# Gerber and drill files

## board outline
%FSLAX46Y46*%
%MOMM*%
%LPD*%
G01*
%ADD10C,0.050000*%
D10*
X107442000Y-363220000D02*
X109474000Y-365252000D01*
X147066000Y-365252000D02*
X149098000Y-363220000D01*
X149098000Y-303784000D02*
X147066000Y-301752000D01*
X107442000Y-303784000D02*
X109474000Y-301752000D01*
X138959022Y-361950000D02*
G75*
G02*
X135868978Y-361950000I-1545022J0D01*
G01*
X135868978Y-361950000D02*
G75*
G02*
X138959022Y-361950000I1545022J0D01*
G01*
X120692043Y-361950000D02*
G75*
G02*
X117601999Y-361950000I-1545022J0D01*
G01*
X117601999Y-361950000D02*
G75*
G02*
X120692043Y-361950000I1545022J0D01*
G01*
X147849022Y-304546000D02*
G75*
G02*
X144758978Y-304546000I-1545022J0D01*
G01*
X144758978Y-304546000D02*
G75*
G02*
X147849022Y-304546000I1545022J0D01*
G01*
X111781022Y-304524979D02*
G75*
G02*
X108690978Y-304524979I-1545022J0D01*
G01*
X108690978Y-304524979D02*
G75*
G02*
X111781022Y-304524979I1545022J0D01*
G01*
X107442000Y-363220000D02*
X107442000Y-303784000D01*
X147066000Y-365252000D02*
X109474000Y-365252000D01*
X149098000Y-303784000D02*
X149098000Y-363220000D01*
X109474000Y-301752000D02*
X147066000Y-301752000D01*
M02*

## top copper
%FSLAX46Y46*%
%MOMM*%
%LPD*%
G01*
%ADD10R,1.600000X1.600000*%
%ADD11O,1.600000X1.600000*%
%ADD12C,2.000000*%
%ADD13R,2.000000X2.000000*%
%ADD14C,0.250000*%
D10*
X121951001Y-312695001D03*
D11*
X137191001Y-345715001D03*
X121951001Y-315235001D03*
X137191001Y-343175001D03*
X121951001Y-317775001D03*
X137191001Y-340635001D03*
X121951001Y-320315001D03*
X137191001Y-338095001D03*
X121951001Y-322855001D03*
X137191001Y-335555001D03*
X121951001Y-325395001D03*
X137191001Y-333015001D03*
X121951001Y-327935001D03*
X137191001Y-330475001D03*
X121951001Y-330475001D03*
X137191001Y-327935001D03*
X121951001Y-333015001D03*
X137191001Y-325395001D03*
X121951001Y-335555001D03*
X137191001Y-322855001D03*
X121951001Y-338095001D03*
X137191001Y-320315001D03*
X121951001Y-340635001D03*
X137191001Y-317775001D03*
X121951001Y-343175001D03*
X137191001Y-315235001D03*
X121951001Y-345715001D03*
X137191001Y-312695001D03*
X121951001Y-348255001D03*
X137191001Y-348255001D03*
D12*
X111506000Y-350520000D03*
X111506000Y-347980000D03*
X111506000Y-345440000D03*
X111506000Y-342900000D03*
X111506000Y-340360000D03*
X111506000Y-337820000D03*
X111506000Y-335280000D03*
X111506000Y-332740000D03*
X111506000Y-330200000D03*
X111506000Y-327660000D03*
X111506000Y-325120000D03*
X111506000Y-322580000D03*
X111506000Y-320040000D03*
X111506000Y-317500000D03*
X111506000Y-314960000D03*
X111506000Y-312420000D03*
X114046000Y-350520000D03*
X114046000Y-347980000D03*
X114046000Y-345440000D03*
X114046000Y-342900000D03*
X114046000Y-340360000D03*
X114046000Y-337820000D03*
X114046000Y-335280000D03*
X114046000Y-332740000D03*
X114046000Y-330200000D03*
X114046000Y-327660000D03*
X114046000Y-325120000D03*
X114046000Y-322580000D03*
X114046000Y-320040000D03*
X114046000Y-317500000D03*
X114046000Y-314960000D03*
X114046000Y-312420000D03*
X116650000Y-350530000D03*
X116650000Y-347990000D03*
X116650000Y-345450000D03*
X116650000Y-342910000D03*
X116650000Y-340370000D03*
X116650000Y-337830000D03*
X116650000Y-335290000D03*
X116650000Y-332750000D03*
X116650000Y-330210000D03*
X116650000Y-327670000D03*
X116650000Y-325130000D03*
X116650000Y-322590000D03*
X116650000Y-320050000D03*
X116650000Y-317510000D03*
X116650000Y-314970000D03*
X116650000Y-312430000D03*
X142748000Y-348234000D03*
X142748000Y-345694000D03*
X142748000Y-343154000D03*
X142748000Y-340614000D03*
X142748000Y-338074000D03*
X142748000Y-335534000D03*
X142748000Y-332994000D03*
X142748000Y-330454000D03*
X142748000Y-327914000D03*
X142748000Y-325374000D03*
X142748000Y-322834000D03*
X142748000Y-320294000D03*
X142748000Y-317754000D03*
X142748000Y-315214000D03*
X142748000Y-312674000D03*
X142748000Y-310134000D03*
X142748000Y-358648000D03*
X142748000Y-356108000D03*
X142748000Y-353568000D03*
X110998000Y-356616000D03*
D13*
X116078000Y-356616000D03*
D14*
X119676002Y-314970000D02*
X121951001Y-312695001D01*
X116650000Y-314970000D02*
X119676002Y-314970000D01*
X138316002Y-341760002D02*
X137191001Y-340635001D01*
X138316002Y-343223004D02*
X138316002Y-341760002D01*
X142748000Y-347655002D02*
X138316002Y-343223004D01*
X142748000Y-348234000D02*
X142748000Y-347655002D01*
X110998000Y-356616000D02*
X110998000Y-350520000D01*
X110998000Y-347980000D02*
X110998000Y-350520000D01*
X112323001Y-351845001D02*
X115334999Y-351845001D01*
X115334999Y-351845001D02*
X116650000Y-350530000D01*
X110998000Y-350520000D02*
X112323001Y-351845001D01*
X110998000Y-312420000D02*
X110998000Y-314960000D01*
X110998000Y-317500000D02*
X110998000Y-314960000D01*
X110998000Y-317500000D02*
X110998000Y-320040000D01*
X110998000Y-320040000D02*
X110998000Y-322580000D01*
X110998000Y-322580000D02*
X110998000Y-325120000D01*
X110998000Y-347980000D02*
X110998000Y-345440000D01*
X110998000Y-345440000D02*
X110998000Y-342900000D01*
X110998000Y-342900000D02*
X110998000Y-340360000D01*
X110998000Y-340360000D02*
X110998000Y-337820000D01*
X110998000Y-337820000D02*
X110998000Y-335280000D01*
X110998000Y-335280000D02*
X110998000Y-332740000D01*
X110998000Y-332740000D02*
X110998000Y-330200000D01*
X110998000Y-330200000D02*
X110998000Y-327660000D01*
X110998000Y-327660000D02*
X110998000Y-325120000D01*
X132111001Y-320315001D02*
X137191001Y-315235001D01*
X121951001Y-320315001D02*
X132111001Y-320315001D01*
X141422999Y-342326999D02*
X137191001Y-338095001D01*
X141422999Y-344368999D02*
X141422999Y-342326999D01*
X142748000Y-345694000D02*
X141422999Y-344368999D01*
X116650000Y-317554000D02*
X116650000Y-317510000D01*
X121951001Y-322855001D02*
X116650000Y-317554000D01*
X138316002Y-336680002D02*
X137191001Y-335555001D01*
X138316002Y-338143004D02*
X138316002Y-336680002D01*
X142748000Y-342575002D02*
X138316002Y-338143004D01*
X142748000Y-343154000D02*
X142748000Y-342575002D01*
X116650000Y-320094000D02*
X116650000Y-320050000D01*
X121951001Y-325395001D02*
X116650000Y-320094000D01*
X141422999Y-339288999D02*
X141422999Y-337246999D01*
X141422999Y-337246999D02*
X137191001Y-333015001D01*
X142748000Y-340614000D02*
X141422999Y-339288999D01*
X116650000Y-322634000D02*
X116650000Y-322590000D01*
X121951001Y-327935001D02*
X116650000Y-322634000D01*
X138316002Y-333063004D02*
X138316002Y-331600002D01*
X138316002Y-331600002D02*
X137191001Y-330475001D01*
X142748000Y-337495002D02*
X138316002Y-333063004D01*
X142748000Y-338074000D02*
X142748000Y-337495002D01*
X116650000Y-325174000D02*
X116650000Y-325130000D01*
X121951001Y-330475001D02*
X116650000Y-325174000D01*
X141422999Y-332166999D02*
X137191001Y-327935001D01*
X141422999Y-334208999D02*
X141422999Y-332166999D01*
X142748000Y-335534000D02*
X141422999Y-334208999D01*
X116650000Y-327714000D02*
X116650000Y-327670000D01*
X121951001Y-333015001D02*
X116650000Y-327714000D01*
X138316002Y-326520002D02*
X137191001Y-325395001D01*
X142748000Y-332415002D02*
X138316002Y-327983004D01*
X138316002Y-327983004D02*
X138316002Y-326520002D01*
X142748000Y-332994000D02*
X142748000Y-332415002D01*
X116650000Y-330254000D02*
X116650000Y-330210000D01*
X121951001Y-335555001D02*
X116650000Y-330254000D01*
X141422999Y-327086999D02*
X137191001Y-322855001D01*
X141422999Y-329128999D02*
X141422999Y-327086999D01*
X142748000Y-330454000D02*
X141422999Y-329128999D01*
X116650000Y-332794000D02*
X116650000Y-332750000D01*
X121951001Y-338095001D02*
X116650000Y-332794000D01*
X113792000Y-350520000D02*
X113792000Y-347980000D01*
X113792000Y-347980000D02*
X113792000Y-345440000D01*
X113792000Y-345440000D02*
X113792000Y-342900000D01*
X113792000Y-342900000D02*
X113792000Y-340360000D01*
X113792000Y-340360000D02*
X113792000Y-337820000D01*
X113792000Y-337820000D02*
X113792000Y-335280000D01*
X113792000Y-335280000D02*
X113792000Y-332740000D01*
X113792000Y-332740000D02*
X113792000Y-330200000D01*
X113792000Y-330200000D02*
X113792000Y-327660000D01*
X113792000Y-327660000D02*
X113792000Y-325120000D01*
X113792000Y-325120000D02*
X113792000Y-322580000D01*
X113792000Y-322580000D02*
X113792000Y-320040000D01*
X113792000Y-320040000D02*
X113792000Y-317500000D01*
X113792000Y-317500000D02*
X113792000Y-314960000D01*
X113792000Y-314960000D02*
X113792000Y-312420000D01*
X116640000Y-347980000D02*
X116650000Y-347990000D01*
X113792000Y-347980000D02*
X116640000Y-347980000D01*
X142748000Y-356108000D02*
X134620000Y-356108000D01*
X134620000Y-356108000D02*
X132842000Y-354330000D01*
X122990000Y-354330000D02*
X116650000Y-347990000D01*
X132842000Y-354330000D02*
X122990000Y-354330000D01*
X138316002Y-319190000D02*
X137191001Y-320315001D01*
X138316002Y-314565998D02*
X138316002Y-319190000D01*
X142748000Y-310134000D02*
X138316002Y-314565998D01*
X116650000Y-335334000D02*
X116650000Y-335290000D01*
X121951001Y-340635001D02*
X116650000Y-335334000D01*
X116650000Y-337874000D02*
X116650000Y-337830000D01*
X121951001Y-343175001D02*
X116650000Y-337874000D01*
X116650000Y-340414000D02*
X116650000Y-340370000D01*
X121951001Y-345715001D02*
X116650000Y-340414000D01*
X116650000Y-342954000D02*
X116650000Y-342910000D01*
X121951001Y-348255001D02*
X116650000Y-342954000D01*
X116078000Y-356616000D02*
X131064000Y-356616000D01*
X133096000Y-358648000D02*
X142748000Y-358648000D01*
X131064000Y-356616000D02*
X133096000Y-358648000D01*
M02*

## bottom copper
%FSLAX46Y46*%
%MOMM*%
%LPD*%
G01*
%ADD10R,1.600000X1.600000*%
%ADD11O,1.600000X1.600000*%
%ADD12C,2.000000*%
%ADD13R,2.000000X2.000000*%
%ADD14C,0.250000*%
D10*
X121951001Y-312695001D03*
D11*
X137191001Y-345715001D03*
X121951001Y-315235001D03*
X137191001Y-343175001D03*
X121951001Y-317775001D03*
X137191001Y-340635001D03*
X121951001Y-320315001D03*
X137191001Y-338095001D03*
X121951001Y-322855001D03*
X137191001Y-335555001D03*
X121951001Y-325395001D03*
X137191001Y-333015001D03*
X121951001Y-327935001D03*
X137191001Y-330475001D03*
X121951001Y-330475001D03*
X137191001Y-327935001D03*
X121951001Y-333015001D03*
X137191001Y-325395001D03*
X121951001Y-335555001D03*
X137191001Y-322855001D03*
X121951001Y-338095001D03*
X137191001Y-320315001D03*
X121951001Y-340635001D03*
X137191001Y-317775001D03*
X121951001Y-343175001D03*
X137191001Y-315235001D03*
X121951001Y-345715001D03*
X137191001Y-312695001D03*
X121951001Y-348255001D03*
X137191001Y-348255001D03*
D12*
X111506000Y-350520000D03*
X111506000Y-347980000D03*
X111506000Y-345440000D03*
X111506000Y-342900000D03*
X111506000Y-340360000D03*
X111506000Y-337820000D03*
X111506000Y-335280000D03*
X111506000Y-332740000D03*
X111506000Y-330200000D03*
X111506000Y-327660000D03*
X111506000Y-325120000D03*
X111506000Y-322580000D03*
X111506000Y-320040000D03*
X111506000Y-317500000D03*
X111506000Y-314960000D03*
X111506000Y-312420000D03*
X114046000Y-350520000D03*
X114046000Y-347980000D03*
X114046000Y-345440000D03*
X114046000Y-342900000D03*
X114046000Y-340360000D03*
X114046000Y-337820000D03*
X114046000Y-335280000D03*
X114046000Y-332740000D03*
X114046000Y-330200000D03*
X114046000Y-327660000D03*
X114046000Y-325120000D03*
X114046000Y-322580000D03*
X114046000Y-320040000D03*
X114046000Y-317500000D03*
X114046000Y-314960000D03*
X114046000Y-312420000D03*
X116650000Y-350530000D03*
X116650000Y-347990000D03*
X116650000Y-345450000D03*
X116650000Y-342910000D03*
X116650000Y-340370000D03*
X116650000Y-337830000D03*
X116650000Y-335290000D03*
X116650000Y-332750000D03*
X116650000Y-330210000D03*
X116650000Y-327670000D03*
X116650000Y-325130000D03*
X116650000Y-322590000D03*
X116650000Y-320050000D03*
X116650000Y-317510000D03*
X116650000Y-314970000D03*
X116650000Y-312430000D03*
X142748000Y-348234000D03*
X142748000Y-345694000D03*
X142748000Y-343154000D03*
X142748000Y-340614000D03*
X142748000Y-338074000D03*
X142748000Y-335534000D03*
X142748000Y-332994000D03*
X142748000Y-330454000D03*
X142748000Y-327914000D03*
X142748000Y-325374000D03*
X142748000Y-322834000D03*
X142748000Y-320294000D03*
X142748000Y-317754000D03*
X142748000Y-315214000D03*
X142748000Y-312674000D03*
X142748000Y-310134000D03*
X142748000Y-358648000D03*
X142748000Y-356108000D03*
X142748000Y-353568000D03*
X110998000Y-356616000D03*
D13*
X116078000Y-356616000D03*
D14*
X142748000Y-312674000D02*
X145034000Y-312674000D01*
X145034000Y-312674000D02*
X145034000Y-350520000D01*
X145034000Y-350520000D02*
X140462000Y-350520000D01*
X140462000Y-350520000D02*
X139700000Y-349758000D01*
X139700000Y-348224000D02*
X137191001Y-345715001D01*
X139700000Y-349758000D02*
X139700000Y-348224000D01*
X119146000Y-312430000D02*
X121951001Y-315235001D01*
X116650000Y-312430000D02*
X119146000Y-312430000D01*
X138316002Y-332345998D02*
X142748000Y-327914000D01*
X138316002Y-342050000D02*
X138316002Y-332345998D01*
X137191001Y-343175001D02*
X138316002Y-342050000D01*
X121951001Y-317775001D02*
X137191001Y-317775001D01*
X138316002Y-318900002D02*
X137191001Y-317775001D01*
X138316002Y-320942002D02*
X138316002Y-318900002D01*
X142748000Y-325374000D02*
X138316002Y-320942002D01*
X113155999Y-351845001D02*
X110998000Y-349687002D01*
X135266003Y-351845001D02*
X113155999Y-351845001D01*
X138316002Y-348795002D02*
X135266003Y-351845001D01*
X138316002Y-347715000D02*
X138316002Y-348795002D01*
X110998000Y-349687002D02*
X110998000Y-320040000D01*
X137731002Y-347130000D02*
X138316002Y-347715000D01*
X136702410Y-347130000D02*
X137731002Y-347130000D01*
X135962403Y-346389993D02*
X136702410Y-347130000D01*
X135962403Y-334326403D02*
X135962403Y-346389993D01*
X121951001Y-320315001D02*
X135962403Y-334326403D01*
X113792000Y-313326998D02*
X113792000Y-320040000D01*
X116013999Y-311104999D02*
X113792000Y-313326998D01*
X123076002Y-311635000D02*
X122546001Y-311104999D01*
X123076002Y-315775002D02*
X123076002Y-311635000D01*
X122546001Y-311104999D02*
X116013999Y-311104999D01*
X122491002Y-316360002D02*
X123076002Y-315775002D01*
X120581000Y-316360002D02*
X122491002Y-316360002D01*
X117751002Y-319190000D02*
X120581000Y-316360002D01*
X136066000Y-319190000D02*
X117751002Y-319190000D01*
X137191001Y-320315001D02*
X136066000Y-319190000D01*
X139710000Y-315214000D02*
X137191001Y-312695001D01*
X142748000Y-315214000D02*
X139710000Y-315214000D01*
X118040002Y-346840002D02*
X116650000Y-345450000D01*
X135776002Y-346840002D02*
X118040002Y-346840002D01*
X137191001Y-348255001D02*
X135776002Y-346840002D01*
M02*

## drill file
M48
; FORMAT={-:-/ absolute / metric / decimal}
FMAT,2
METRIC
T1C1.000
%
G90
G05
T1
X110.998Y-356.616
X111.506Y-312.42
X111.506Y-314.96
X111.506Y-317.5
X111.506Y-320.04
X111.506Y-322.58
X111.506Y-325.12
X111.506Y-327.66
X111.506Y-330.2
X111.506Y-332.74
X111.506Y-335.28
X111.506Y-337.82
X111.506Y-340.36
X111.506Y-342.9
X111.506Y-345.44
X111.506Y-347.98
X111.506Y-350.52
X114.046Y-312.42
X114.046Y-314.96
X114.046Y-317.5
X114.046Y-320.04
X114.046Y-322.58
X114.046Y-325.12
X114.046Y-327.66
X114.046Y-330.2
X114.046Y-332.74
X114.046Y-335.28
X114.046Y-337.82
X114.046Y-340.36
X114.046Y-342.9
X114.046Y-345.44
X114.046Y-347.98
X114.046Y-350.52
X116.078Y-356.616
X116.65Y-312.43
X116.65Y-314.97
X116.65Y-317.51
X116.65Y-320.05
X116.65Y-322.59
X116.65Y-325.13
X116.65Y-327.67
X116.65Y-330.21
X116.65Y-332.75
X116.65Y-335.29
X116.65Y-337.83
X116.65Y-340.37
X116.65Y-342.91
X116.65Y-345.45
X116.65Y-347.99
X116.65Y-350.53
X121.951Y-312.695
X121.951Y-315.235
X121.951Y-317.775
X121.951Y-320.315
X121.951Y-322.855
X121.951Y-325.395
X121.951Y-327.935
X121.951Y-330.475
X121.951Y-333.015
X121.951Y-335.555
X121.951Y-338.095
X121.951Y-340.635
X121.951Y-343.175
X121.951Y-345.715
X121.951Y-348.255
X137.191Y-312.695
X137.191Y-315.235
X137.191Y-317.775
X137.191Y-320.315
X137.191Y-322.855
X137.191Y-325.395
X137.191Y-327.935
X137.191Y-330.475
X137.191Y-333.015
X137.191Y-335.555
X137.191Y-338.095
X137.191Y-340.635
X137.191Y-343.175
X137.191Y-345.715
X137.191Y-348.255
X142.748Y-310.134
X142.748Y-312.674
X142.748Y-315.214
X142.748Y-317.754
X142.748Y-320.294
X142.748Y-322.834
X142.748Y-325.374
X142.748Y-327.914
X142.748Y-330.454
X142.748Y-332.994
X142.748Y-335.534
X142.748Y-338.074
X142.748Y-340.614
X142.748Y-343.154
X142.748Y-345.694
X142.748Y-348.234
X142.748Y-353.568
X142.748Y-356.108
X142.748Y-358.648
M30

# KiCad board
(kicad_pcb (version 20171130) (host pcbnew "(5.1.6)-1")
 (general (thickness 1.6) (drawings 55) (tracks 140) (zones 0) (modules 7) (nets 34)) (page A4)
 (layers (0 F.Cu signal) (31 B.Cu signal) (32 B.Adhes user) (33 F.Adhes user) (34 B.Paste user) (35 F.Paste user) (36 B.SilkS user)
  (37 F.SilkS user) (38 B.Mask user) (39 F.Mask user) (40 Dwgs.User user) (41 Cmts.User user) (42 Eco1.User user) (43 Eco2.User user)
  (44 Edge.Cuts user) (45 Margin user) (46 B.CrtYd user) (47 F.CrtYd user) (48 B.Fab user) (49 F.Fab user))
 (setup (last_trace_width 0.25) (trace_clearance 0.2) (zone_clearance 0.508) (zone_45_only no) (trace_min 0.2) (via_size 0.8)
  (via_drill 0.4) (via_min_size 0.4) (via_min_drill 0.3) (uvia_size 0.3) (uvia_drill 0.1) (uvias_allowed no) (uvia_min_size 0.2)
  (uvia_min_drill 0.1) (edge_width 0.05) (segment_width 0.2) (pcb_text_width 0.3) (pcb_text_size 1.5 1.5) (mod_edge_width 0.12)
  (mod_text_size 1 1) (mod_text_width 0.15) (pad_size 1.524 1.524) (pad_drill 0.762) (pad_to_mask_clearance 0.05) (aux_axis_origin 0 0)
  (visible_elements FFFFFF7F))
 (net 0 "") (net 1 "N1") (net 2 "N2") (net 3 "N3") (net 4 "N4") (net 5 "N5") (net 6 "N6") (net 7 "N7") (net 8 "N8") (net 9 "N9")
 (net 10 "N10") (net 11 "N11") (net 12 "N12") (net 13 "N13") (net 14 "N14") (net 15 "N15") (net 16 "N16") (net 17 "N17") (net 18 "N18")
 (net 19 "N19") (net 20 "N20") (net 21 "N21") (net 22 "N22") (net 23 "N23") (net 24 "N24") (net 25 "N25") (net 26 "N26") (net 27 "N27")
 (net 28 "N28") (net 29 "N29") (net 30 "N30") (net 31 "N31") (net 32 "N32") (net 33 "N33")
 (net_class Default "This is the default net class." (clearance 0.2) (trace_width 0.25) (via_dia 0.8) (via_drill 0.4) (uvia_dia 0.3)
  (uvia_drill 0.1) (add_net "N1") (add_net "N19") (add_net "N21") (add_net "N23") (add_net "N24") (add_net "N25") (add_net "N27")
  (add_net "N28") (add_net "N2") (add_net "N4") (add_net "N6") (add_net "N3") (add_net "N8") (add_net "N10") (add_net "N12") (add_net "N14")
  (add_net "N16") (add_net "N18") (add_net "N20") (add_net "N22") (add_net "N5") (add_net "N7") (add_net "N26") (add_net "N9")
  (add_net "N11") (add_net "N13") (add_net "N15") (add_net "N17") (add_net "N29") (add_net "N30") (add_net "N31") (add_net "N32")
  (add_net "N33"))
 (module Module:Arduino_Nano (layer F.Cu) (at 121.951001 312.695001)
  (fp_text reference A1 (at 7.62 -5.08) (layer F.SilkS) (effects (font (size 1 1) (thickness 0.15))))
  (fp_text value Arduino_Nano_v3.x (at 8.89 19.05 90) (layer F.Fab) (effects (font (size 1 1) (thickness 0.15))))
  (pad 1 thru_hole rect (at 0 0) (size 1.6 1.6) (drill 1) (layers *.Cu *.Mask) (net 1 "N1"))
  (pad 17 thru_hole oval (at 15.24 33.02) (size 1.6 1.6) (drill 1) (layers *.Cu *.Mask) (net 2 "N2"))
  (pad 2 thru_hole oval (at 0 2.54) (size 1.6 1.6) (drill 1) (layers *.Cu *.Mask) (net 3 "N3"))
  (pad 18 thru_hole oval (at 15.24 30.48) (size 1.6 1.6) (drill 1) (layers *.Cu *.Mask) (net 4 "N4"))
  (pad 3 thru_hole oval (at 0 5.08) (size 1.6 1.6) (drill 1) (layers *.Cu *.Mask) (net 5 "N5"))
  (pad 19 thru_hole oval (at 15.24 27.94) (size 1.6 1.6) (drill 1) (layers *.Cu *.Mask) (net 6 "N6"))
  (pad 4 thru_hole oval (at 0 7.62) (size 1.6 1.6) (drill 1) (layers *.Cu *.Mask) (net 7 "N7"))
  (pad 20 thru_hole oval (at 15.24 25.4) (size 1.6 1.6) (drill 1) (layers *.Cu *.Mask) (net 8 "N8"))
  (pad 5 thru_hole oval (at 0 10.16) (size 1.6 1.6) (drill 1) (layers *.Cu *.Mask) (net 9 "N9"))
  (pad 21 thru_hole oval (at 15.24 22.86) (size 1.6 1.6) (drill 1) (layers *.Cu *.Mask) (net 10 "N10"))
  (pad 6 thru_hole oval (at 0 12.7) (size 1.6 1.6) (drill 1) (layers *.Cu *.Mask) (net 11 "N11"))
  (pad 22 thru_hole oval (at 15.24 20.32) (size 1.6 1.6) (drill 1) (layers *.Cu *.Mask) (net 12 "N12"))
  (pad 7 thru_hole oval (at 0 15.24) (size 1.6 1.6) (drill 1) (layers *.Cu *.Mask) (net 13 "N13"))
  (pad 23 thru_hole oval (at 15.24 17.78) (size 1.6 1.6) (drill 1) (layers *.Cu *.Mask) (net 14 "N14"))
  (pad 8 thru_hole oval (at 0 17.78) (size 1.6 1.6) (drill 1) (layers *.Cu *.Mask) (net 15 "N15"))
  (pad 24 thru_hole oval (at 15.24 15.24) (size 1.6 1.6) (drill 1) (layers *.Cu *.Mask) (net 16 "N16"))
  (pad 9 thru_hole oval (at 0 20.32) (size 1.6 1.6) (drill 1) (layers *.Cu *.Mask) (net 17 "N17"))
  (pad 25 thru_hole oval (at 15.24 12.7) (size 1.6 1.6) (drill 1) (layers *.Cu *.Mask) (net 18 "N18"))
  (pad 10 thru_hole oval (at 0 22.86) (size 1.6 1.6) (drill 1) (layers *.Cu *.Mask) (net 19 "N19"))
  (pad 26 thru_hole oval (at 15.24 10.16) (size 1.6 1.6) (drill 1) (layers *.Cu *.Mask) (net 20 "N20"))
  (pad 11 thru_hole oval (at 0 25.4) (size 1.6 1.6) (drill 1) (layers *.Cu *.Mask) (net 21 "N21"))
  (pad 27 thru_hole oval (at 15.24 7.62) (size 1.6 1.6) (drill 1) (layers *.Cu *.Mask) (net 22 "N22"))
  (pad 12 thru_hole oval (at 0 27.94) (size 1.6 1.6) (drill 1) (layers *.Cu *.Mask) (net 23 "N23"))
  (pad 28 thru_hole oval (at 15.24 5.08) (size 1.6 1.6) (drill 1) (layers *.Cu *.Mask) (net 5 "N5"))
  (pad 13 thru_hole oval (at 0 30.48) (size 1.6 1.6) (drill 1) (layers *.Cu *.Mask) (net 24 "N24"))
  (pad 29 thru_hole oval (at 15.24 2.54) (size 1.6 1.6) (drill 1) (layers *.Cu *.Mask) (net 7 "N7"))
  (pad 14 thru_hole oval (at 0 33.02) (size 1.6 1.6) (drill 1) (layers *.Cu *.Mask) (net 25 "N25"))
  (pad 30 thru_hole oval (at 15.24 0) (size 1.6 1.6) (drill 1) (layers *.Cu *.Mask) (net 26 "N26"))
  (pad 15 thru_hole oval (at 0 35.56) (size 1.6 1.6) (drill 1) (layers *.Cu *.Mask) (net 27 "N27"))
  (pad 16 thru_hole oval (at 15.24 35.56) (size 1.6 1.6) (drill 1) (layers *.Cu *.Mask) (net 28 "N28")))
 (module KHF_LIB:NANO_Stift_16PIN (layer F.Cu) (at 111.506 350.52 90)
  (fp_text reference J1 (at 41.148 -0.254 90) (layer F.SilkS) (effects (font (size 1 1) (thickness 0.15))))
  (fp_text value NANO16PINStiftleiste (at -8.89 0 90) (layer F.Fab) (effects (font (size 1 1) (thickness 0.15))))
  (pad 1 thru_hole circle (at 0 0 90) (size 2 2) (drill 1) (layers *.Cu *.Mask) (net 7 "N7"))
  (pad 2 thru_hole circle (at 2.54 0 90) (size 2 2) (drill 1) (layers *.Cu *.Mask) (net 7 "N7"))
  (pad 3 thru_hole circle (at 5.08 0 90) (size 2 2) (drill 1) (layers *.Cu *.Mask) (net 7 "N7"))
  (pad 4 thru_hole circle (at 7.62 0 90) (size 2 2) (drill 1) (layers *.Cu *.Mask) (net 7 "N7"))
  (pad 5 thru_hole circle (at 10.16 0 90) (size 2 2) (drill 1) (layers *.Cu *.Mask) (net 7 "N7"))
  (pad 6 thru_hole circle (at 12.7 0 90) (size 2 2) (drill 1) (layers *.Cu *.Mask) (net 7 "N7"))
  (pad 7 thru_hole circle (at 15.24 0 90) (size 2 2) (drill 1) (layers *.Cu *.Mask) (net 7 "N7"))
  (pad 8 thru_hole circle (at 17.78 0 90) (size 2 2) (drill 1) (layers *.Cu *.Mask) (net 7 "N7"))
  (pad 9 thru_hole circle (at 20.32 0 90) (size 2 2) (drill 1) (layers *.Cu *.Mask) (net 7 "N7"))
  (pad 10 thru_hole circle (at 22.86 0 90) (size 2 2) (drill 1) (layers *.Cu *.Mask) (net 7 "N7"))
  (pad 11 thru_hole circle (at 25.4 0 90) (size 2 2) (drill 1) (layers *.Cu *.Mask) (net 7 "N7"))
  (pad 12 thru_hole circle (at 27.94 0 90) (size 2 2) (drill 1) (layers *.Cu *.Mask) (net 7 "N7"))
  (pad 13 thru_hole circle (at 30.48 0 90) (size 2 2) (drill 1) (layers *.Cu *.Mask) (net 7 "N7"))
  (pad 14 thru_hole circle (at 33.02 0 90) (size 2 2) (drill 1) (layers *.Cu *.Mask) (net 7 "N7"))
  (pad 15 thru_hole circle (at 35.56 0 90) (size 2 2) (drill 1) (layers *.Cu *.Mask) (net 7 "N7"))
  (pad 16 thru_hole circle (at 38.1 0 90) (size 2 2) (drill 1) (layers *.Cu *.Mask) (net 7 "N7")))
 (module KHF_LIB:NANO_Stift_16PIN (layer F.Cu) (at 114.046 312.42 270)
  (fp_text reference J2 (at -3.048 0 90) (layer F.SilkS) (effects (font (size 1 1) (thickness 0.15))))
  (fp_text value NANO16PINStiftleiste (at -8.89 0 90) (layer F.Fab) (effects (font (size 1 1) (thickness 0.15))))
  (pad 16 thru_hole circle (at 38.1 0 270) (size 2 2) (drill 1) (layers *.Cu *.Mask) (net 22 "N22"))
  (pad 15 thru_hole circle (at 35.56 0 270) (size 2 2) (drill 1) (layers *.Cu *.Mask) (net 22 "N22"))
  (pad 14 thru_hole circle (at 33.02 0 270) (size 2 2) (drill 1) (layers *.Cu *.Mask) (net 22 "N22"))
  (pad 13 thru_hole circle (at 30.48 0 270) (size 2 2) (drill 1) (layers *.Cu *.Mask) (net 22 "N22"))
  (pad 12 thru_hole circle (at 27.94 0 270) (size 2 2) (drill 1) (layers *.Cu *.Mask) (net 22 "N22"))
  (pad 11 thru_hole circle (at 25.4 0 270) (size 2 2) (drill 1) (layers *.Cu *.Mask) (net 22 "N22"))
  (pad 10 thru_hole circle (at 22.86 0 270) (size 2 2) (drill 1) (layers *.Cu *.Mask) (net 22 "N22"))
  (pad 9 thru_hole circle (at 20.32 0 270) (size 2 2) (drill 1) (layers *.Cu *.Mask) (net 22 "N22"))
  (pad 8 thru_hole circle (at 17.78 0 270) (size 2 2) (drill 1) (layers *.Cu *.Mask) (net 22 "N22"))
  (pad 7 thru_hole circle (at 15.24 0 270) (size 2 2) (drill 1) (layers *.Cu *.Mask) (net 22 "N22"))
  (pad 6 thru_hole circle (at 12.7 0 270) (size 2 2) (drill 1) (layers *.Cu *.Mask) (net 22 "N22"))
  (pad 5 thru_hole circle (at 10.16 0 270) (size 2 2) (drill 1) (layers *.Cu *.Mask) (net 22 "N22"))
  (pad 4 thru_hole circle (at 7.62 0 270) (size 2 2) (drill 1) (layers *.Cu *.Mask) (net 22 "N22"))
  (pad 3 thru_hole circle (at 5.08 0 270) (size 2 2) (drill 1) (layers *.Cu *.Mask) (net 22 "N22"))
  (pad 2 thru_hole circle (at 2.54 0 270) (size 2 2) (drill 1) (layers *.Cu *.Mask) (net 22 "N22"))
  (pad 1 thru_hole circle (at 0 0 270) (size 2 2) (drill 1) (layers *.Cu *.Mask) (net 22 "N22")))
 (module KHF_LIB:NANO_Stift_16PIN (layer F.Cu) (at 116.65 312.43 270)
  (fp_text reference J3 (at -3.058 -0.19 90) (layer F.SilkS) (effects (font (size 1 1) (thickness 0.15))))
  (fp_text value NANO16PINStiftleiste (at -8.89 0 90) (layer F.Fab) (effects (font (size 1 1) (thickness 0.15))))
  (pad 16 thru_hole circle (at 38.1 0 270) (size 2 2) (drill 1) (layers *.Cu *.Mask) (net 7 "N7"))
  (pad 15 thru_hole circle (at 35.56 0 270) (size 2 2) (drill 1) (layers *.Cu *.Mask) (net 22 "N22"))
  (pad 14 thru_hole circle (at 33.02 0 270) (size 2 2) (drill 1) (layers *.Cu *.Mask) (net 28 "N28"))
  (pad 13 thru_hole circle (at 30.48 0 270) (size 2 2) (drill 1) (layers *.Cu *.Mask) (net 27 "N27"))
  (pad 12 thru_hole circle (at 27.94 0 270) (size 2 2) (drill 1) (layers *.Cu *.Mask) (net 25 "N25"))
  (pad 11 thru_hole circle (at 25.4 0 270) (size 2 2) (drill 1) (layers *.Cu *.Mask) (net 24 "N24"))
  (pad 10 thru_hole circle (at 22.86 0 270) (size 2 2) (drill 1) (layers *.Cu *.Mask) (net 23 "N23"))
  (pad 9 thru_hole circle (at 20.32 0 270) (size 2 2) (drill 1) (layers *.Cu *.Mask) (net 21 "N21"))
  (pad 8 thru_hole circle (at 17.78 0 270) (size 2 2) (drill 1) (layers *.Cu *.Mask) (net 19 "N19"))
  (pad 7 thru_hole circle (at 15.24 0 270) (size 2 2) (drill 1) (layers *.Cu *.Mask) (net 17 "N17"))
  (pad 6 thru_hole circle (at 12.7 0 270) (size 2 2) (drill 1) (layers *.Cu *.Mask) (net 15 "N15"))
  (pad 5 thru_hole circle (at 10.16 0 270) (size 2 2) (drill 1) (layers *.Cu *.Mask) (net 13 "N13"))
  (pad 4 thru_hole circle (at 7.62 0 270) (size 2 2) (drill 1) (layers *.Cu *.Mask) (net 11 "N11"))
  (pad 3 thru_hole circle (at 5.08 0 270) (size 2 2) (drill 1) (layers *.Cu *.Mask) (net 9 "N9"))
  (pad 2 thru_hole circle (at 2.54 0 270) (size 2 2) (drill 1) (layers *.Cu *.Mask) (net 1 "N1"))
  (pad 1 thru_hole circle (at 0 0 270) (size 2 2) (drill 1) (layers *.Cu *.Mask) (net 3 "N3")))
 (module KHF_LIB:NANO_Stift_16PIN (layer F.Cu) (at 142.748 348.234 90)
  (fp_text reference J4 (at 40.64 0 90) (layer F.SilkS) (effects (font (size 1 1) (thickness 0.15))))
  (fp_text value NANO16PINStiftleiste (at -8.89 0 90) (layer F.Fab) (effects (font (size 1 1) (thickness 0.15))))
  (pad 1 thru_hole circle (at 0 0 90) (size 2 2) (drill 1) (layers *.Cu *.Mask) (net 6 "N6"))
  (pad 2 thru_hole circle (at 2.54 0 90) (size 2 2) (drill 1) (layers *.Cu *.Mask) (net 8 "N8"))
  (pad 3 thru_hole circle (at 5.08 0 90) (size 2 2) (drill 1) (layers *.Cu *.Mask) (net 10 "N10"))
  (pad 4 thru_hole circle (at 7.62 0 90) (size 2 2) (drill 1) (layers *.Cu *.Mask) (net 12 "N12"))
  (pad 5 thru_hole circle (at 10.16 0 90) (size 2 2) (drill 1) (layers *.Cu *.Mask) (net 14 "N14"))
  (pad 6 thru_hole circle (at 12.7 0 90) (size 2 2) (drill 1) (layers *.Cu *.Mask) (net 16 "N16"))
  (pad 7 thru_hole circle (at 15.24 0 90) (size 2 2) (drill 1) (layers *.Cu *.Mask) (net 18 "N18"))
  (pad 8 thru_hole circle (at 17.78 0 90) (size 2 2) (drill 1) (layers *.Cu *.Mask) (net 20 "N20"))
  (pad 9 thru_hole circle (at 20.32 0 90) (size 2 2) (drill 1) (layers *.Cu *.Mask) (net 4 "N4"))
  (pad 10 thru_hole circle (at 22.86 0 90) (size 2 2) (drill 1) (layers *.Cu *.Mask) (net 5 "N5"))
  (pad 11 thru_hole circle (at 25.4 0 90) (size 2 2) (drill 1) (layers *.Cu *.Mask) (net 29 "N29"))
  (pad 12 thru_hole circle (at 27.94 0 90) (size 2 2) (drill 1) (layers *.Cu *.Mask) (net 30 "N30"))
  (pad 13 thru_hole circle (at 30.48 0 90) (size 2 2) (drill 1) (layers *.Cu *.Mask) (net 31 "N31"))
  (pad 14 thru_hole circle (at 33.02 0 90) (size 2 2) (drill 1) (layers *.Cu *.Mask) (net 26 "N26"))
  (pad 15 thru_hole circle (at 35.56 0 90) (size 2 2) (drill 1) (layers *.Cu *.Mask) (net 2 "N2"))
  (pad 16 thru_hole circle (at 38.1 0 90) (size 2 2) (drill 1) (layers *.Cu *.Mask) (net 22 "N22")))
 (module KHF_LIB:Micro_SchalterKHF (layer F.Cu) (at 142.748 358.648 90)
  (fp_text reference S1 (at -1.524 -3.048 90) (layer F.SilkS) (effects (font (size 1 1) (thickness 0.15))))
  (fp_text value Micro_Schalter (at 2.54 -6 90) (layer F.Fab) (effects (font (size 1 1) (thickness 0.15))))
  (pad 1 thru_hole circle (at 0 0 90) (size 2 2) (drill 1) (layers *.Cu *.Mask) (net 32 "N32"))
  (pad 2 thru_hole circle (at 2.54 0 90) (size 2 2) (drill 1) (layers *.Cu *.Mask) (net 22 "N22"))
  (pad 3 thru_hole circle (at 5.08 0 90) (size 2 2) (drill 1) (layers *.Cu *.Mask) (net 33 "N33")))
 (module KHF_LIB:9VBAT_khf (layer F.Cu) (at 110.998 356.616)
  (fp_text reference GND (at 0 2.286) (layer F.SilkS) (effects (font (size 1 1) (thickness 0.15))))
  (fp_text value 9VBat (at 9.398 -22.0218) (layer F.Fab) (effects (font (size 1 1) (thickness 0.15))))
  (pad 1 thru_hole circle (at 0 0) (size 2 2) (drill 1) (layers *.Cu *.Mask) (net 7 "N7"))
  (pad 2 thru_hole rect (at 5.08 0) (size 2 2) (drill 1) (layers *.Cu *.Mask) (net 32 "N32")))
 (gr_line (start 107.442 363.22) (end 109.474 365.252) (layer Edge.Cuts) (width 0.05))
 (gr_line (start 147.066 365.252) (end 149.098 363.22) (layer Edge.Cuts) (width 0.05))
 (gr_line (start 149.098 303.784) (end 147.066 301.752) (layer Edge.Cuts) (width 0.05))
 (gr_line (start 107.442 303.784) (end 109.474 301.752) (layer Edge.Cuts) (width 0.05))
 (gr_circle (center 137.414 361.95) (end 138.938 361.696) (layer Edge.Cuts) (width 0.05))
 (gr_circle (center 119.147021 361.95) (end 120.671021 361.696) (layer Edge.Cuts) (width 0.05))
 (gr_circle (center 146.304 304.546) (end 147.828 304.292) (layer Edge.Cuts) (width 0.05))
 (gr_circle (center 110.236 304.524979) (end 111.76 304.270979) (layer Edge.Cuts) (width 0.05))
 (gr_line (start 107.442 363.22) (end 107.442 303.784) (layer Edge.Cuts) (width 0.05))
 (gr_line (start 147.066 365.252) (end 109.474 365.252) (layer Edge.Cuts) (width 0.05))
 (gr_line (start 149.098 303.784) (end 149.098 363.22) (layer Edge.Cuts) (width 0.05))
 (gr_line (start 109.474 301.752) (end 147.066 301.752) (layer Edge.Cuts) (width 0.05))
 (segment (start 119.676002 314.97) (end 121.951001 312.695001) (width 0.25) (layer F.Cu) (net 1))
 (segment (start 116.65 314.97) (end 119.676002 314.97) (width 0.25) (layer F.Cu) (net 1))
 (segment (start 142.748 312.674) (end 145.034 312.674) (width 0.25) (layer B.Cu) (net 2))
 (segment (start 145.034 312.674) (end 145.034 350.52) (width 0.25) (layer B.Cu) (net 2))
 (segment (start 145.034 350.52) (end 140.462 350.52) (width 0.25) (layer B.Cu) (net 2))
 (segment (start 140.462 350.52) (end 139.7 349.758) (width 0.25) (layer B.Cu) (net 2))
 (segment (start 139.7 348.224) (end 137.191001 345.715001) (width 0.25) (layer B.Cu) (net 2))
 (segment (start 139.7 349.758) (end 139.7 348.224) (width 0.25) (layer B.Cu) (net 2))
 (segment (start 119.146 312.43) (end 121.951001 315.235001) (width 0.25) (layer B.Cu) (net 3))
 (segment (start 116.65 312.43) (end 119.146 312.43) (width 0.25) (layer B.Cu) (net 3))
 (segment (start 138.316002 332.345998) (end 142.748 327.914) (width 0.25) (layer B.Cu) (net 4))
 (segment (start 138.316002 342.05) (end 138.316002 332.345998) (width 0.25) (layer B.Cu) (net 4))
 (segment (start 137.191001 343.175001) (end 138.316002 342.05) (width 0.25) (layer B.Cu) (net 4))
 (segment (start 121.951001 317.775001) (end 137.191001 317.775001) (width 0.25) (layer B.Cu) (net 5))
 (segment (start 138.316002 318.900002) (end 137.191001 317.775001) (width 0.25) (layer B.Cu) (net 5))
 (segment (start 138.316002 320.942002) (end 138.316002 318.900002) (width 0.25) (layer B.Cu) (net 5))
 (segment (start 142.748 325.374) (end 138.316002 320.942002) (width 0.25) (layer B.Cu) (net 5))
 (segment (start 138.316002 341.760002) (end 137.191001 340.635001) (width 0.25) (layer F.Cu) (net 6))
 (segment (start 138.316002 343.223004) (end 138.316002 341.760002) (width 0.25) (layer F.Cu) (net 6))
 (segment (start 142.748 347.655002) (end 138.316002 343.223004) (width 0.25) (layer F.Cu) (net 6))
 (segment (start 142.748 348.234) (end 142.748 347.655002) (width 0.25) (layer F.Cu) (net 6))
 (segment (start 110.998 356.616) (end 110.998 350.52) (width 0.25) (layer F.Cu) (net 7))
 (segment (start 110.998 347.98) (end 110.998 350.52) (width 0.25) (layer F.Cu) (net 7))
 (segment (start 112.323001 351.845001) (end 115.334999 351.845001) (width 0.25) (layer F.Cu) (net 7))
 (segment (start 115.334999 351.845001) (end 116.65 350.53) (width 0.25) (layer F.Cu) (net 7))
 (segment (start 110.998 350.52) (end 112.323001 351.845001) (width 0.25) (layer F.Cu) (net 7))
 (segment (start 110.998 312.42) (end 110.998 314.96) (width 0.25) (layer F.Cu) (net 7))
 (segment (start 110.998 317.5) (end 110.998 314.96) (width 0.25) (layer F.Cu) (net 7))
 (segment (start 110.998 317.5) (end 110.998 320.04) (width 0.25) (layer F.Cu) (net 7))
 (segment (start 110.998 320.04) (end 110.998 322.58) (width 0.25) (layer F.Cu) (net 7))
 (segment (start 110.998 322.58) (end 110.998 325.12) (width 0.25) (layer F.Cu) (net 7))
 (segment (start 110.998 347.98) (end 110.998 345.44) (width 0.25) (layer F.Cu) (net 7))
 (segment (start 110.998 345.44) (end 110.998 342.9) (width 0.25) (layer F.Cu) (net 7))
 (segment (start 110.998 342.9) (end 110.998 340.36) (width 0.25) (layer F.Cu) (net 7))
 (segment (start 110.998 340.36) (end 110.998 337.82) (width 0.25) (layer F.Cu) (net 7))
 (segment (start 110.998 337.82) (end 110.998 335.28) (width 0.25) (layer F.Cu) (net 7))
 (segment (start 110.998 335.28) (end 110.998 332.74) (width 0.25) (layer F.Cu) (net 7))
 (segment (start 110.998 332.74) (end 110.998 330.2) (width 0.25) (layer F.Cu) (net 7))
 (segment (start 110.998 330.2) (end 110.998 327.66) (width 0.25) (layer F.Cu) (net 7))
 (segment (start 110.998 327.66) (end 110.998 325.12) (width 0.25) (layer F.Cu) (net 7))
 (segment (start 132.111001 320.315001) (end 137.191001 315.235001) (width 0.25) (layer F.Cu) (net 7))
 (segment (start 121.951001 320.315001) (end 132.111001 320.315001) (width 0.25) (layer F.Cu) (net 7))
 (segment (start 113.155999 351.845001) (end 110.998 349.687002) (width 0.25) (layer B.Cu) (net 7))
 (segment (start 135.266003 351.845001) (end 113.155999 351.845001) (width 0.25) (layer B.Cu) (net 7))
 (segment (start 138.316002 348.795002) (end 135.266003 351.845001) (width 0.25) (layer B.Cu) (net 7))
 (segment (start 138.316002 347.715) (end 138.316002 348.795002) (width 0.25) (layer B.Cu) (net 7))
 (segment (start 110.998 349.687002) (end 110.998 320.04) (width 0.25) (layer B.Cu) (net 7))
 (segment (start 137.731002 347.13) (end 138.316002 347.715) (width 0.25) (layer B.Cu) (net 7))
 (segment (start 136.70241 347.13) (end 137.731002 347.13) (width 0.25) (layer B.Cu) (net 7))
 (segment (start 135.962403 346.389993) (end 136.70241 347.13) (width 0.25) (layer B.Cu) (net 7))
 (segment (start 135.962403 334.326403) (end 135.962403 346.389993) (width 0.25) (layer B.Cu) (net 7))
 (segment (start 121.951001 320.315001) (end 135.962403 334.326403) (width 0.25) (layer B.Cu) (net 7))
 (segment (start 141.422999 342.326999) (end 137.191001 338.095001) (width 0.25) (layer F.Cu) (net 8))
 (segment (start 141.422999 344.368999) (end 141.422999 342.326999) (width 0.25) (layer F.Cu) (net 8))
 (segment (start 142.748 345.694) (end 141.422999 344.368999) (width 0.25) (layer F.Cu) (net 8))
 (segment (start 116.65 317.554) (end 116.65 317.51) (width 0.25) (layer F.Cu) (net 9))
 (segment (start 121.951001 322.855001) (end 116.65 317.554) (width 0.25) (layer F.Cu) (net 9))
 (segment (start 138.316002 336.680002) (end 137.191001 335.555001) (width 0.25) (layer F.Cu) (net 10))
 (segment (start 138.316002 338.143004) (end 138.316002 336.680002) (width 0.25) (layer F.Cu) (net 10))
 (segment (start 142.748 342.575002) (end 138.316002 338.143004) (width 0.25) (layer F.Cu) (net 10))
 (segment (start 142.748 343.154) (end 142.748 342.575002) (width 0.25) (layer F.Cu) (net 10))
 (segment (start 116.65 320.094) (end 116.65 320.05) (width 0.25) (layer F.Cu) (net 11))
 (segment (start 121.951001 325.395001) (end 116.65 320.094) (width 0.25) (layer F.Cu) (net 11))
 (segment (start 141.422999 339.288999) (end 141.422999 337.246999) (width 0.25) (layer F.Cu) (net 12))
 (segment (start 141.422999 337.246999) (end 137.191001 333.015001) (width 0.25) (layer F.Cu) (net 12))
 (segment (start 142.748 340.614) (end 141.422999 339.288999) (width 0.25) (layer F.Cu) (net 12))
 (segment (start 116.65 322.634) (end 116.65 322.59) (width 0.25) (layer F.Cu) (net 13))
 (segment (start 121.951001 327.935001) (end 116.65 322.634) (width 0.25) (layer F.Cu) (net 13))
 (segment (start 138.316002 333.063004) (end 138.316002 331.600002) (width 0.25) (layer F.Cu) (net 14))
 (segment (start 138.316002 331.600002) (end 137.191001 330.475001) (width 0.25) (layer F.Cu) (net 14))
 (segment (start 142.748 337.495002) (end 138.316002 333.063004) (width 0.25) (layer F.Cu) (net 14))
 (segment (start 142.748 338.074) (end 142.748 337.495002) (width 0.25) (layer F.Cu) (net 14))
 (segment (start 116.65 325.174) (end 116.65 325.13) (width 0.25) (layer F.Cu) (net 15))
 (segment (start 121.951001 330.475001) (end 116.65 325.174) (width 0.25) (layer F.Cu) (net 15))
 (segment (start 141.422999 332.166999) (end 137.191001 327.935001) (width 0.25) (layer F.Cu) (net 16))
 (segment (start 141.422999 334.208999) (end 141.422999 332.166999) (width 0.25) (layer F.Cu) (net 16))
 (segment (start 142.748 335.534) (end 141.422999 334.208999) (width 0.25) (layer F.Cu) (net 16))
 (segment (start 116.65 327.714) (end 116.65 327.67) (width 0.25) (layer F.Cu) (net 17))
 (segment (start 121.951001 333.015001) (end 116.65 327.714) (width 0.25) (layer F.Cu) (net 17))
 (segment (start 138.316002 326.520002) (end 137.191001 325.395001) (width 0.25) (layer F.Cu) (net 18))
 (segment (start 142.748 332.415002) (end 138.316002 327.983004) (width 0.25) (layer F.Cu) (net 18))
 (segment (start 138.316002 327.983004) (end 138.316002 326.520002) (width 0.25) (layer F.Cu) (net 18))
 (segment (start 142.748 332.994) (end 142.748 332.415002) (width 0.25) (layer F.Cu) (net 18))
 (segment (start 116.65 330.254) (end 116.65 330.21) (width 0.25) (layer F.Cu) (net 19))
 (segment (start 121.951001 335.555001) (end 116.65 330.254) (width 0.25) (layer F.Cu) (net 19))
 (segment (start 141.422999 327.086999) (end 137.191001 322.855001) (width 0.25) (layer F.Cu) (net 20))
 (segment (start 141.422999 329.128999) (end 141.422999 327.086999) (width 0.25) (layer F.Cu) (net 20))
 (segment (start 142.748 330.454) (end 141.422999 329.128999) (width 0.25) (layer F.Cu) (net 20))
 (segment (start 116.65 332.794) (end 116.65 332.75) (width 0.25) (layer F.Cu) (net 21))
 (segment (start 121.951001 338.095001) (end 116.65 332.794) (width 0.25) (layer F.Cu) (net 21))
 (segment (start 113.792 350.52) (end 113.792 347.98) (width 0.25) (layer F.Cu) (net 22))
 (segment (start 113.792 347.98) (end 113.792 345.44) (width 0.25) (layer F.Cu) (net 22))
 (segment (start 113.792 345.44) (end 113.792 342.9) (width 0.25) (layer F.Cu) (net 22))
 (segment (start 113.792 342.9) (end 113.792 340.36) (width 0.25) (layer F.Cu) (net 22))
 (segment (start 113.792 340.36) (end 113.792 337.82) (width 0.25) (layer F.Cu) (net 22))
 (segment (start 113.792 337.82) (end 113.792 335.28) (width 0.25) (layer F.Cu) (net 22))
 (segment (start 113.792 335.28) (end 113.792 332.74) (width 0.25) (layer F.Cu) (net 22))
 (segment (start 113.792 332.74) (end 113.792 330.2) (width 0.25) (layer F.Cu) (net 22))
 (segment (start 113.792 330.2) (end 113.792 327.66) (width 0.25) (layer F.Cu) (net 22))
 (segment (start 113.792 327.66) (end 113.792 325.12) (width 0.25) (layer F.Cu) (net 22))
 (segment (start 113.792 325.12) (end 113.792 322.58) (width 0.25) (layer F.Cu) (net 22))
 (segment (start 113.792 322.58) (end 113.792 320.04) (width 0.25) (layer F.Cu) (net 22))
 (segment (start 113.792 320.04) (end 113.792 317.5) (width 0.25) (layer F.Cu) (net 22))
 (segment (start 113.792 317.5) (end 113.792 314.96) (width 0.25) (layer F.Cu) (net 22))
 (segment (start 113.792 314.96) (end 113.792 312.42) (width 0.25) (layer F.Cu) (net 22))
 (segment (start 116.64 347.98) (end 116.65 347.99) (width 0.25) (layer F.Cu) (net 22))
 (segment (start 113.792 347.98) (end 116.64 347.98) (width 0.25) (layer F.Cu) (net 22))
 (segment (start 142.748 356.108) (end 134.62 356.108) (width 0.25) (layer F.Cu) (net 22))
 (segment (start 134.62 356.108) (end 132.842 354.33) (width 0.25) (layer F.Cu) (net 22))
 (segment (start 122.99 354.33) (end 116.65 347.99) (width 0.25) (layer F.Cu) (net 22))
 (segment (start 132.842 354.33) (end 122.99 354.33) (width 0.25) (layer F.Cu) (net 22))
 (segment (start 138.316002 319.19) (end 137.191001 320.315001) (width 0.25) (layer F.Cu) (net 22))
 (segment (start 138.316002 314.565998) (end 138.316002 319.19) (width 0.25) (layer F.Cu) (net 22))
 (segment (start 142.748 310.134) (end 138.316002 314.565998) (width 0.25) (layer F.Cu) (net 22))
 (segment (start 113.792 313.326998) (end 113.792 320.04) (width 0.25) (layer B.Cu) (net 22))
 (segment (start 116.013999 311.104999) (end 113.792 313.326998) (width 0.25) (layer B.Cu) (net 22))
 (segment (start 123.076002 311.635) (end 122.546001 311.104999) (width 0.25) (layer B.Cu) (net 22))
 (segment (start 123.076002 315.775002) (end 123.076002 311.635) (width 0.25) (layer B.Cu) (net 22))
 (segment (start 122.546001 311.104999) (end 116.013999 311.104999) (width 0.25) (layer B.Cu) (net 22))
 (segment (start 122.491002 316.360002) (end 123.076002 315.775002) (width 0.25) (layer B.Cu) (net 22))
 (segment (start 120.581 316.360002) (end 122.491002 316.360002) (width 0.25) (layer B.Cu) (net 22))
 (segment (start 117.751002 319.19) (end 120.581 316.360002) (width 0.25) (layer B.Cu) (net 22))
 (segment (start 136.066 319.19) (end 117.751002 319.19) (width 0.25) (layer B.Cu) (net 22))
 (segment (start 137.191001 320.315001) (end 136.066 319.19) (width 0.25) (layer B.Cu) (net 22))
 (segment (start 116.65 335.334) (end 116.65 335.29) (width 0.25) (layer F.Cu) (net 23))
 (segment (start 121.951001 340.635001) (end 116.65 335.334) (width 0.25) (layer F.Cu) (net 23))
 (segment (start 116.65 337.874) (end 116.65 337.83) (width 0.25) (layer F.Cu) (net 24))
 (segment (start 121.951001 343.175001) (end 116.65 337.874) (width 0.25) (layer F.Cu) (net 24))
 (segment (start 116.65 340.414) (end 116.65 340.37) (width 0.25) (layer F.Cu) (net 25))
 (segment (start 121.951001 345.715001) (end 116.65 340.414) (width 0.25) (layer F.Cu) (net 25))
 (segment (start 139.71 315.214) (end 137.191001 312.695001) (width 0.25) (layer B.Cu) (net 26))
 (segment (start 142.748 315.214) (end 139.71 315.214) (width 0.25) (layer B.Cu) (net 26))
 (segment (start 116.65 342.954) (end 116.65 342.91) (width 0.25) (layer F.Cu) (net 27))
 (segment (start 121.951001 348.255001) (end 116.65 342.954) (width 0.25) (layer F.Cu) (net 27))
 (segment (start 118.040002 346.840002) (end 116.65 345.45) (width 0.25) (layer B.Cu) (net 28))
 (segment (start 135.776002 346.840002) (end 118.040002 346.840002) (width 0.25) (layer B.Cu) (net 28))
 (segment (start 137.191001 348.255001) (end 135.776002 346.840002) (width 0.25) (layer B.Cu) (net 28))
 (segment (start 116.078 356.616) (end 131.064 356.616) (width 0.25) (layer F.Cu) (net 32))
 (segment (start 133.096 358.648) (end 142.748 358.648) (width 0.25) (layer F.Cu) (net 32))
 (segment (start 131.064 356.616) (end 133.096 358.648) (width 0.25) (layer F.Cu) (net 32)))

